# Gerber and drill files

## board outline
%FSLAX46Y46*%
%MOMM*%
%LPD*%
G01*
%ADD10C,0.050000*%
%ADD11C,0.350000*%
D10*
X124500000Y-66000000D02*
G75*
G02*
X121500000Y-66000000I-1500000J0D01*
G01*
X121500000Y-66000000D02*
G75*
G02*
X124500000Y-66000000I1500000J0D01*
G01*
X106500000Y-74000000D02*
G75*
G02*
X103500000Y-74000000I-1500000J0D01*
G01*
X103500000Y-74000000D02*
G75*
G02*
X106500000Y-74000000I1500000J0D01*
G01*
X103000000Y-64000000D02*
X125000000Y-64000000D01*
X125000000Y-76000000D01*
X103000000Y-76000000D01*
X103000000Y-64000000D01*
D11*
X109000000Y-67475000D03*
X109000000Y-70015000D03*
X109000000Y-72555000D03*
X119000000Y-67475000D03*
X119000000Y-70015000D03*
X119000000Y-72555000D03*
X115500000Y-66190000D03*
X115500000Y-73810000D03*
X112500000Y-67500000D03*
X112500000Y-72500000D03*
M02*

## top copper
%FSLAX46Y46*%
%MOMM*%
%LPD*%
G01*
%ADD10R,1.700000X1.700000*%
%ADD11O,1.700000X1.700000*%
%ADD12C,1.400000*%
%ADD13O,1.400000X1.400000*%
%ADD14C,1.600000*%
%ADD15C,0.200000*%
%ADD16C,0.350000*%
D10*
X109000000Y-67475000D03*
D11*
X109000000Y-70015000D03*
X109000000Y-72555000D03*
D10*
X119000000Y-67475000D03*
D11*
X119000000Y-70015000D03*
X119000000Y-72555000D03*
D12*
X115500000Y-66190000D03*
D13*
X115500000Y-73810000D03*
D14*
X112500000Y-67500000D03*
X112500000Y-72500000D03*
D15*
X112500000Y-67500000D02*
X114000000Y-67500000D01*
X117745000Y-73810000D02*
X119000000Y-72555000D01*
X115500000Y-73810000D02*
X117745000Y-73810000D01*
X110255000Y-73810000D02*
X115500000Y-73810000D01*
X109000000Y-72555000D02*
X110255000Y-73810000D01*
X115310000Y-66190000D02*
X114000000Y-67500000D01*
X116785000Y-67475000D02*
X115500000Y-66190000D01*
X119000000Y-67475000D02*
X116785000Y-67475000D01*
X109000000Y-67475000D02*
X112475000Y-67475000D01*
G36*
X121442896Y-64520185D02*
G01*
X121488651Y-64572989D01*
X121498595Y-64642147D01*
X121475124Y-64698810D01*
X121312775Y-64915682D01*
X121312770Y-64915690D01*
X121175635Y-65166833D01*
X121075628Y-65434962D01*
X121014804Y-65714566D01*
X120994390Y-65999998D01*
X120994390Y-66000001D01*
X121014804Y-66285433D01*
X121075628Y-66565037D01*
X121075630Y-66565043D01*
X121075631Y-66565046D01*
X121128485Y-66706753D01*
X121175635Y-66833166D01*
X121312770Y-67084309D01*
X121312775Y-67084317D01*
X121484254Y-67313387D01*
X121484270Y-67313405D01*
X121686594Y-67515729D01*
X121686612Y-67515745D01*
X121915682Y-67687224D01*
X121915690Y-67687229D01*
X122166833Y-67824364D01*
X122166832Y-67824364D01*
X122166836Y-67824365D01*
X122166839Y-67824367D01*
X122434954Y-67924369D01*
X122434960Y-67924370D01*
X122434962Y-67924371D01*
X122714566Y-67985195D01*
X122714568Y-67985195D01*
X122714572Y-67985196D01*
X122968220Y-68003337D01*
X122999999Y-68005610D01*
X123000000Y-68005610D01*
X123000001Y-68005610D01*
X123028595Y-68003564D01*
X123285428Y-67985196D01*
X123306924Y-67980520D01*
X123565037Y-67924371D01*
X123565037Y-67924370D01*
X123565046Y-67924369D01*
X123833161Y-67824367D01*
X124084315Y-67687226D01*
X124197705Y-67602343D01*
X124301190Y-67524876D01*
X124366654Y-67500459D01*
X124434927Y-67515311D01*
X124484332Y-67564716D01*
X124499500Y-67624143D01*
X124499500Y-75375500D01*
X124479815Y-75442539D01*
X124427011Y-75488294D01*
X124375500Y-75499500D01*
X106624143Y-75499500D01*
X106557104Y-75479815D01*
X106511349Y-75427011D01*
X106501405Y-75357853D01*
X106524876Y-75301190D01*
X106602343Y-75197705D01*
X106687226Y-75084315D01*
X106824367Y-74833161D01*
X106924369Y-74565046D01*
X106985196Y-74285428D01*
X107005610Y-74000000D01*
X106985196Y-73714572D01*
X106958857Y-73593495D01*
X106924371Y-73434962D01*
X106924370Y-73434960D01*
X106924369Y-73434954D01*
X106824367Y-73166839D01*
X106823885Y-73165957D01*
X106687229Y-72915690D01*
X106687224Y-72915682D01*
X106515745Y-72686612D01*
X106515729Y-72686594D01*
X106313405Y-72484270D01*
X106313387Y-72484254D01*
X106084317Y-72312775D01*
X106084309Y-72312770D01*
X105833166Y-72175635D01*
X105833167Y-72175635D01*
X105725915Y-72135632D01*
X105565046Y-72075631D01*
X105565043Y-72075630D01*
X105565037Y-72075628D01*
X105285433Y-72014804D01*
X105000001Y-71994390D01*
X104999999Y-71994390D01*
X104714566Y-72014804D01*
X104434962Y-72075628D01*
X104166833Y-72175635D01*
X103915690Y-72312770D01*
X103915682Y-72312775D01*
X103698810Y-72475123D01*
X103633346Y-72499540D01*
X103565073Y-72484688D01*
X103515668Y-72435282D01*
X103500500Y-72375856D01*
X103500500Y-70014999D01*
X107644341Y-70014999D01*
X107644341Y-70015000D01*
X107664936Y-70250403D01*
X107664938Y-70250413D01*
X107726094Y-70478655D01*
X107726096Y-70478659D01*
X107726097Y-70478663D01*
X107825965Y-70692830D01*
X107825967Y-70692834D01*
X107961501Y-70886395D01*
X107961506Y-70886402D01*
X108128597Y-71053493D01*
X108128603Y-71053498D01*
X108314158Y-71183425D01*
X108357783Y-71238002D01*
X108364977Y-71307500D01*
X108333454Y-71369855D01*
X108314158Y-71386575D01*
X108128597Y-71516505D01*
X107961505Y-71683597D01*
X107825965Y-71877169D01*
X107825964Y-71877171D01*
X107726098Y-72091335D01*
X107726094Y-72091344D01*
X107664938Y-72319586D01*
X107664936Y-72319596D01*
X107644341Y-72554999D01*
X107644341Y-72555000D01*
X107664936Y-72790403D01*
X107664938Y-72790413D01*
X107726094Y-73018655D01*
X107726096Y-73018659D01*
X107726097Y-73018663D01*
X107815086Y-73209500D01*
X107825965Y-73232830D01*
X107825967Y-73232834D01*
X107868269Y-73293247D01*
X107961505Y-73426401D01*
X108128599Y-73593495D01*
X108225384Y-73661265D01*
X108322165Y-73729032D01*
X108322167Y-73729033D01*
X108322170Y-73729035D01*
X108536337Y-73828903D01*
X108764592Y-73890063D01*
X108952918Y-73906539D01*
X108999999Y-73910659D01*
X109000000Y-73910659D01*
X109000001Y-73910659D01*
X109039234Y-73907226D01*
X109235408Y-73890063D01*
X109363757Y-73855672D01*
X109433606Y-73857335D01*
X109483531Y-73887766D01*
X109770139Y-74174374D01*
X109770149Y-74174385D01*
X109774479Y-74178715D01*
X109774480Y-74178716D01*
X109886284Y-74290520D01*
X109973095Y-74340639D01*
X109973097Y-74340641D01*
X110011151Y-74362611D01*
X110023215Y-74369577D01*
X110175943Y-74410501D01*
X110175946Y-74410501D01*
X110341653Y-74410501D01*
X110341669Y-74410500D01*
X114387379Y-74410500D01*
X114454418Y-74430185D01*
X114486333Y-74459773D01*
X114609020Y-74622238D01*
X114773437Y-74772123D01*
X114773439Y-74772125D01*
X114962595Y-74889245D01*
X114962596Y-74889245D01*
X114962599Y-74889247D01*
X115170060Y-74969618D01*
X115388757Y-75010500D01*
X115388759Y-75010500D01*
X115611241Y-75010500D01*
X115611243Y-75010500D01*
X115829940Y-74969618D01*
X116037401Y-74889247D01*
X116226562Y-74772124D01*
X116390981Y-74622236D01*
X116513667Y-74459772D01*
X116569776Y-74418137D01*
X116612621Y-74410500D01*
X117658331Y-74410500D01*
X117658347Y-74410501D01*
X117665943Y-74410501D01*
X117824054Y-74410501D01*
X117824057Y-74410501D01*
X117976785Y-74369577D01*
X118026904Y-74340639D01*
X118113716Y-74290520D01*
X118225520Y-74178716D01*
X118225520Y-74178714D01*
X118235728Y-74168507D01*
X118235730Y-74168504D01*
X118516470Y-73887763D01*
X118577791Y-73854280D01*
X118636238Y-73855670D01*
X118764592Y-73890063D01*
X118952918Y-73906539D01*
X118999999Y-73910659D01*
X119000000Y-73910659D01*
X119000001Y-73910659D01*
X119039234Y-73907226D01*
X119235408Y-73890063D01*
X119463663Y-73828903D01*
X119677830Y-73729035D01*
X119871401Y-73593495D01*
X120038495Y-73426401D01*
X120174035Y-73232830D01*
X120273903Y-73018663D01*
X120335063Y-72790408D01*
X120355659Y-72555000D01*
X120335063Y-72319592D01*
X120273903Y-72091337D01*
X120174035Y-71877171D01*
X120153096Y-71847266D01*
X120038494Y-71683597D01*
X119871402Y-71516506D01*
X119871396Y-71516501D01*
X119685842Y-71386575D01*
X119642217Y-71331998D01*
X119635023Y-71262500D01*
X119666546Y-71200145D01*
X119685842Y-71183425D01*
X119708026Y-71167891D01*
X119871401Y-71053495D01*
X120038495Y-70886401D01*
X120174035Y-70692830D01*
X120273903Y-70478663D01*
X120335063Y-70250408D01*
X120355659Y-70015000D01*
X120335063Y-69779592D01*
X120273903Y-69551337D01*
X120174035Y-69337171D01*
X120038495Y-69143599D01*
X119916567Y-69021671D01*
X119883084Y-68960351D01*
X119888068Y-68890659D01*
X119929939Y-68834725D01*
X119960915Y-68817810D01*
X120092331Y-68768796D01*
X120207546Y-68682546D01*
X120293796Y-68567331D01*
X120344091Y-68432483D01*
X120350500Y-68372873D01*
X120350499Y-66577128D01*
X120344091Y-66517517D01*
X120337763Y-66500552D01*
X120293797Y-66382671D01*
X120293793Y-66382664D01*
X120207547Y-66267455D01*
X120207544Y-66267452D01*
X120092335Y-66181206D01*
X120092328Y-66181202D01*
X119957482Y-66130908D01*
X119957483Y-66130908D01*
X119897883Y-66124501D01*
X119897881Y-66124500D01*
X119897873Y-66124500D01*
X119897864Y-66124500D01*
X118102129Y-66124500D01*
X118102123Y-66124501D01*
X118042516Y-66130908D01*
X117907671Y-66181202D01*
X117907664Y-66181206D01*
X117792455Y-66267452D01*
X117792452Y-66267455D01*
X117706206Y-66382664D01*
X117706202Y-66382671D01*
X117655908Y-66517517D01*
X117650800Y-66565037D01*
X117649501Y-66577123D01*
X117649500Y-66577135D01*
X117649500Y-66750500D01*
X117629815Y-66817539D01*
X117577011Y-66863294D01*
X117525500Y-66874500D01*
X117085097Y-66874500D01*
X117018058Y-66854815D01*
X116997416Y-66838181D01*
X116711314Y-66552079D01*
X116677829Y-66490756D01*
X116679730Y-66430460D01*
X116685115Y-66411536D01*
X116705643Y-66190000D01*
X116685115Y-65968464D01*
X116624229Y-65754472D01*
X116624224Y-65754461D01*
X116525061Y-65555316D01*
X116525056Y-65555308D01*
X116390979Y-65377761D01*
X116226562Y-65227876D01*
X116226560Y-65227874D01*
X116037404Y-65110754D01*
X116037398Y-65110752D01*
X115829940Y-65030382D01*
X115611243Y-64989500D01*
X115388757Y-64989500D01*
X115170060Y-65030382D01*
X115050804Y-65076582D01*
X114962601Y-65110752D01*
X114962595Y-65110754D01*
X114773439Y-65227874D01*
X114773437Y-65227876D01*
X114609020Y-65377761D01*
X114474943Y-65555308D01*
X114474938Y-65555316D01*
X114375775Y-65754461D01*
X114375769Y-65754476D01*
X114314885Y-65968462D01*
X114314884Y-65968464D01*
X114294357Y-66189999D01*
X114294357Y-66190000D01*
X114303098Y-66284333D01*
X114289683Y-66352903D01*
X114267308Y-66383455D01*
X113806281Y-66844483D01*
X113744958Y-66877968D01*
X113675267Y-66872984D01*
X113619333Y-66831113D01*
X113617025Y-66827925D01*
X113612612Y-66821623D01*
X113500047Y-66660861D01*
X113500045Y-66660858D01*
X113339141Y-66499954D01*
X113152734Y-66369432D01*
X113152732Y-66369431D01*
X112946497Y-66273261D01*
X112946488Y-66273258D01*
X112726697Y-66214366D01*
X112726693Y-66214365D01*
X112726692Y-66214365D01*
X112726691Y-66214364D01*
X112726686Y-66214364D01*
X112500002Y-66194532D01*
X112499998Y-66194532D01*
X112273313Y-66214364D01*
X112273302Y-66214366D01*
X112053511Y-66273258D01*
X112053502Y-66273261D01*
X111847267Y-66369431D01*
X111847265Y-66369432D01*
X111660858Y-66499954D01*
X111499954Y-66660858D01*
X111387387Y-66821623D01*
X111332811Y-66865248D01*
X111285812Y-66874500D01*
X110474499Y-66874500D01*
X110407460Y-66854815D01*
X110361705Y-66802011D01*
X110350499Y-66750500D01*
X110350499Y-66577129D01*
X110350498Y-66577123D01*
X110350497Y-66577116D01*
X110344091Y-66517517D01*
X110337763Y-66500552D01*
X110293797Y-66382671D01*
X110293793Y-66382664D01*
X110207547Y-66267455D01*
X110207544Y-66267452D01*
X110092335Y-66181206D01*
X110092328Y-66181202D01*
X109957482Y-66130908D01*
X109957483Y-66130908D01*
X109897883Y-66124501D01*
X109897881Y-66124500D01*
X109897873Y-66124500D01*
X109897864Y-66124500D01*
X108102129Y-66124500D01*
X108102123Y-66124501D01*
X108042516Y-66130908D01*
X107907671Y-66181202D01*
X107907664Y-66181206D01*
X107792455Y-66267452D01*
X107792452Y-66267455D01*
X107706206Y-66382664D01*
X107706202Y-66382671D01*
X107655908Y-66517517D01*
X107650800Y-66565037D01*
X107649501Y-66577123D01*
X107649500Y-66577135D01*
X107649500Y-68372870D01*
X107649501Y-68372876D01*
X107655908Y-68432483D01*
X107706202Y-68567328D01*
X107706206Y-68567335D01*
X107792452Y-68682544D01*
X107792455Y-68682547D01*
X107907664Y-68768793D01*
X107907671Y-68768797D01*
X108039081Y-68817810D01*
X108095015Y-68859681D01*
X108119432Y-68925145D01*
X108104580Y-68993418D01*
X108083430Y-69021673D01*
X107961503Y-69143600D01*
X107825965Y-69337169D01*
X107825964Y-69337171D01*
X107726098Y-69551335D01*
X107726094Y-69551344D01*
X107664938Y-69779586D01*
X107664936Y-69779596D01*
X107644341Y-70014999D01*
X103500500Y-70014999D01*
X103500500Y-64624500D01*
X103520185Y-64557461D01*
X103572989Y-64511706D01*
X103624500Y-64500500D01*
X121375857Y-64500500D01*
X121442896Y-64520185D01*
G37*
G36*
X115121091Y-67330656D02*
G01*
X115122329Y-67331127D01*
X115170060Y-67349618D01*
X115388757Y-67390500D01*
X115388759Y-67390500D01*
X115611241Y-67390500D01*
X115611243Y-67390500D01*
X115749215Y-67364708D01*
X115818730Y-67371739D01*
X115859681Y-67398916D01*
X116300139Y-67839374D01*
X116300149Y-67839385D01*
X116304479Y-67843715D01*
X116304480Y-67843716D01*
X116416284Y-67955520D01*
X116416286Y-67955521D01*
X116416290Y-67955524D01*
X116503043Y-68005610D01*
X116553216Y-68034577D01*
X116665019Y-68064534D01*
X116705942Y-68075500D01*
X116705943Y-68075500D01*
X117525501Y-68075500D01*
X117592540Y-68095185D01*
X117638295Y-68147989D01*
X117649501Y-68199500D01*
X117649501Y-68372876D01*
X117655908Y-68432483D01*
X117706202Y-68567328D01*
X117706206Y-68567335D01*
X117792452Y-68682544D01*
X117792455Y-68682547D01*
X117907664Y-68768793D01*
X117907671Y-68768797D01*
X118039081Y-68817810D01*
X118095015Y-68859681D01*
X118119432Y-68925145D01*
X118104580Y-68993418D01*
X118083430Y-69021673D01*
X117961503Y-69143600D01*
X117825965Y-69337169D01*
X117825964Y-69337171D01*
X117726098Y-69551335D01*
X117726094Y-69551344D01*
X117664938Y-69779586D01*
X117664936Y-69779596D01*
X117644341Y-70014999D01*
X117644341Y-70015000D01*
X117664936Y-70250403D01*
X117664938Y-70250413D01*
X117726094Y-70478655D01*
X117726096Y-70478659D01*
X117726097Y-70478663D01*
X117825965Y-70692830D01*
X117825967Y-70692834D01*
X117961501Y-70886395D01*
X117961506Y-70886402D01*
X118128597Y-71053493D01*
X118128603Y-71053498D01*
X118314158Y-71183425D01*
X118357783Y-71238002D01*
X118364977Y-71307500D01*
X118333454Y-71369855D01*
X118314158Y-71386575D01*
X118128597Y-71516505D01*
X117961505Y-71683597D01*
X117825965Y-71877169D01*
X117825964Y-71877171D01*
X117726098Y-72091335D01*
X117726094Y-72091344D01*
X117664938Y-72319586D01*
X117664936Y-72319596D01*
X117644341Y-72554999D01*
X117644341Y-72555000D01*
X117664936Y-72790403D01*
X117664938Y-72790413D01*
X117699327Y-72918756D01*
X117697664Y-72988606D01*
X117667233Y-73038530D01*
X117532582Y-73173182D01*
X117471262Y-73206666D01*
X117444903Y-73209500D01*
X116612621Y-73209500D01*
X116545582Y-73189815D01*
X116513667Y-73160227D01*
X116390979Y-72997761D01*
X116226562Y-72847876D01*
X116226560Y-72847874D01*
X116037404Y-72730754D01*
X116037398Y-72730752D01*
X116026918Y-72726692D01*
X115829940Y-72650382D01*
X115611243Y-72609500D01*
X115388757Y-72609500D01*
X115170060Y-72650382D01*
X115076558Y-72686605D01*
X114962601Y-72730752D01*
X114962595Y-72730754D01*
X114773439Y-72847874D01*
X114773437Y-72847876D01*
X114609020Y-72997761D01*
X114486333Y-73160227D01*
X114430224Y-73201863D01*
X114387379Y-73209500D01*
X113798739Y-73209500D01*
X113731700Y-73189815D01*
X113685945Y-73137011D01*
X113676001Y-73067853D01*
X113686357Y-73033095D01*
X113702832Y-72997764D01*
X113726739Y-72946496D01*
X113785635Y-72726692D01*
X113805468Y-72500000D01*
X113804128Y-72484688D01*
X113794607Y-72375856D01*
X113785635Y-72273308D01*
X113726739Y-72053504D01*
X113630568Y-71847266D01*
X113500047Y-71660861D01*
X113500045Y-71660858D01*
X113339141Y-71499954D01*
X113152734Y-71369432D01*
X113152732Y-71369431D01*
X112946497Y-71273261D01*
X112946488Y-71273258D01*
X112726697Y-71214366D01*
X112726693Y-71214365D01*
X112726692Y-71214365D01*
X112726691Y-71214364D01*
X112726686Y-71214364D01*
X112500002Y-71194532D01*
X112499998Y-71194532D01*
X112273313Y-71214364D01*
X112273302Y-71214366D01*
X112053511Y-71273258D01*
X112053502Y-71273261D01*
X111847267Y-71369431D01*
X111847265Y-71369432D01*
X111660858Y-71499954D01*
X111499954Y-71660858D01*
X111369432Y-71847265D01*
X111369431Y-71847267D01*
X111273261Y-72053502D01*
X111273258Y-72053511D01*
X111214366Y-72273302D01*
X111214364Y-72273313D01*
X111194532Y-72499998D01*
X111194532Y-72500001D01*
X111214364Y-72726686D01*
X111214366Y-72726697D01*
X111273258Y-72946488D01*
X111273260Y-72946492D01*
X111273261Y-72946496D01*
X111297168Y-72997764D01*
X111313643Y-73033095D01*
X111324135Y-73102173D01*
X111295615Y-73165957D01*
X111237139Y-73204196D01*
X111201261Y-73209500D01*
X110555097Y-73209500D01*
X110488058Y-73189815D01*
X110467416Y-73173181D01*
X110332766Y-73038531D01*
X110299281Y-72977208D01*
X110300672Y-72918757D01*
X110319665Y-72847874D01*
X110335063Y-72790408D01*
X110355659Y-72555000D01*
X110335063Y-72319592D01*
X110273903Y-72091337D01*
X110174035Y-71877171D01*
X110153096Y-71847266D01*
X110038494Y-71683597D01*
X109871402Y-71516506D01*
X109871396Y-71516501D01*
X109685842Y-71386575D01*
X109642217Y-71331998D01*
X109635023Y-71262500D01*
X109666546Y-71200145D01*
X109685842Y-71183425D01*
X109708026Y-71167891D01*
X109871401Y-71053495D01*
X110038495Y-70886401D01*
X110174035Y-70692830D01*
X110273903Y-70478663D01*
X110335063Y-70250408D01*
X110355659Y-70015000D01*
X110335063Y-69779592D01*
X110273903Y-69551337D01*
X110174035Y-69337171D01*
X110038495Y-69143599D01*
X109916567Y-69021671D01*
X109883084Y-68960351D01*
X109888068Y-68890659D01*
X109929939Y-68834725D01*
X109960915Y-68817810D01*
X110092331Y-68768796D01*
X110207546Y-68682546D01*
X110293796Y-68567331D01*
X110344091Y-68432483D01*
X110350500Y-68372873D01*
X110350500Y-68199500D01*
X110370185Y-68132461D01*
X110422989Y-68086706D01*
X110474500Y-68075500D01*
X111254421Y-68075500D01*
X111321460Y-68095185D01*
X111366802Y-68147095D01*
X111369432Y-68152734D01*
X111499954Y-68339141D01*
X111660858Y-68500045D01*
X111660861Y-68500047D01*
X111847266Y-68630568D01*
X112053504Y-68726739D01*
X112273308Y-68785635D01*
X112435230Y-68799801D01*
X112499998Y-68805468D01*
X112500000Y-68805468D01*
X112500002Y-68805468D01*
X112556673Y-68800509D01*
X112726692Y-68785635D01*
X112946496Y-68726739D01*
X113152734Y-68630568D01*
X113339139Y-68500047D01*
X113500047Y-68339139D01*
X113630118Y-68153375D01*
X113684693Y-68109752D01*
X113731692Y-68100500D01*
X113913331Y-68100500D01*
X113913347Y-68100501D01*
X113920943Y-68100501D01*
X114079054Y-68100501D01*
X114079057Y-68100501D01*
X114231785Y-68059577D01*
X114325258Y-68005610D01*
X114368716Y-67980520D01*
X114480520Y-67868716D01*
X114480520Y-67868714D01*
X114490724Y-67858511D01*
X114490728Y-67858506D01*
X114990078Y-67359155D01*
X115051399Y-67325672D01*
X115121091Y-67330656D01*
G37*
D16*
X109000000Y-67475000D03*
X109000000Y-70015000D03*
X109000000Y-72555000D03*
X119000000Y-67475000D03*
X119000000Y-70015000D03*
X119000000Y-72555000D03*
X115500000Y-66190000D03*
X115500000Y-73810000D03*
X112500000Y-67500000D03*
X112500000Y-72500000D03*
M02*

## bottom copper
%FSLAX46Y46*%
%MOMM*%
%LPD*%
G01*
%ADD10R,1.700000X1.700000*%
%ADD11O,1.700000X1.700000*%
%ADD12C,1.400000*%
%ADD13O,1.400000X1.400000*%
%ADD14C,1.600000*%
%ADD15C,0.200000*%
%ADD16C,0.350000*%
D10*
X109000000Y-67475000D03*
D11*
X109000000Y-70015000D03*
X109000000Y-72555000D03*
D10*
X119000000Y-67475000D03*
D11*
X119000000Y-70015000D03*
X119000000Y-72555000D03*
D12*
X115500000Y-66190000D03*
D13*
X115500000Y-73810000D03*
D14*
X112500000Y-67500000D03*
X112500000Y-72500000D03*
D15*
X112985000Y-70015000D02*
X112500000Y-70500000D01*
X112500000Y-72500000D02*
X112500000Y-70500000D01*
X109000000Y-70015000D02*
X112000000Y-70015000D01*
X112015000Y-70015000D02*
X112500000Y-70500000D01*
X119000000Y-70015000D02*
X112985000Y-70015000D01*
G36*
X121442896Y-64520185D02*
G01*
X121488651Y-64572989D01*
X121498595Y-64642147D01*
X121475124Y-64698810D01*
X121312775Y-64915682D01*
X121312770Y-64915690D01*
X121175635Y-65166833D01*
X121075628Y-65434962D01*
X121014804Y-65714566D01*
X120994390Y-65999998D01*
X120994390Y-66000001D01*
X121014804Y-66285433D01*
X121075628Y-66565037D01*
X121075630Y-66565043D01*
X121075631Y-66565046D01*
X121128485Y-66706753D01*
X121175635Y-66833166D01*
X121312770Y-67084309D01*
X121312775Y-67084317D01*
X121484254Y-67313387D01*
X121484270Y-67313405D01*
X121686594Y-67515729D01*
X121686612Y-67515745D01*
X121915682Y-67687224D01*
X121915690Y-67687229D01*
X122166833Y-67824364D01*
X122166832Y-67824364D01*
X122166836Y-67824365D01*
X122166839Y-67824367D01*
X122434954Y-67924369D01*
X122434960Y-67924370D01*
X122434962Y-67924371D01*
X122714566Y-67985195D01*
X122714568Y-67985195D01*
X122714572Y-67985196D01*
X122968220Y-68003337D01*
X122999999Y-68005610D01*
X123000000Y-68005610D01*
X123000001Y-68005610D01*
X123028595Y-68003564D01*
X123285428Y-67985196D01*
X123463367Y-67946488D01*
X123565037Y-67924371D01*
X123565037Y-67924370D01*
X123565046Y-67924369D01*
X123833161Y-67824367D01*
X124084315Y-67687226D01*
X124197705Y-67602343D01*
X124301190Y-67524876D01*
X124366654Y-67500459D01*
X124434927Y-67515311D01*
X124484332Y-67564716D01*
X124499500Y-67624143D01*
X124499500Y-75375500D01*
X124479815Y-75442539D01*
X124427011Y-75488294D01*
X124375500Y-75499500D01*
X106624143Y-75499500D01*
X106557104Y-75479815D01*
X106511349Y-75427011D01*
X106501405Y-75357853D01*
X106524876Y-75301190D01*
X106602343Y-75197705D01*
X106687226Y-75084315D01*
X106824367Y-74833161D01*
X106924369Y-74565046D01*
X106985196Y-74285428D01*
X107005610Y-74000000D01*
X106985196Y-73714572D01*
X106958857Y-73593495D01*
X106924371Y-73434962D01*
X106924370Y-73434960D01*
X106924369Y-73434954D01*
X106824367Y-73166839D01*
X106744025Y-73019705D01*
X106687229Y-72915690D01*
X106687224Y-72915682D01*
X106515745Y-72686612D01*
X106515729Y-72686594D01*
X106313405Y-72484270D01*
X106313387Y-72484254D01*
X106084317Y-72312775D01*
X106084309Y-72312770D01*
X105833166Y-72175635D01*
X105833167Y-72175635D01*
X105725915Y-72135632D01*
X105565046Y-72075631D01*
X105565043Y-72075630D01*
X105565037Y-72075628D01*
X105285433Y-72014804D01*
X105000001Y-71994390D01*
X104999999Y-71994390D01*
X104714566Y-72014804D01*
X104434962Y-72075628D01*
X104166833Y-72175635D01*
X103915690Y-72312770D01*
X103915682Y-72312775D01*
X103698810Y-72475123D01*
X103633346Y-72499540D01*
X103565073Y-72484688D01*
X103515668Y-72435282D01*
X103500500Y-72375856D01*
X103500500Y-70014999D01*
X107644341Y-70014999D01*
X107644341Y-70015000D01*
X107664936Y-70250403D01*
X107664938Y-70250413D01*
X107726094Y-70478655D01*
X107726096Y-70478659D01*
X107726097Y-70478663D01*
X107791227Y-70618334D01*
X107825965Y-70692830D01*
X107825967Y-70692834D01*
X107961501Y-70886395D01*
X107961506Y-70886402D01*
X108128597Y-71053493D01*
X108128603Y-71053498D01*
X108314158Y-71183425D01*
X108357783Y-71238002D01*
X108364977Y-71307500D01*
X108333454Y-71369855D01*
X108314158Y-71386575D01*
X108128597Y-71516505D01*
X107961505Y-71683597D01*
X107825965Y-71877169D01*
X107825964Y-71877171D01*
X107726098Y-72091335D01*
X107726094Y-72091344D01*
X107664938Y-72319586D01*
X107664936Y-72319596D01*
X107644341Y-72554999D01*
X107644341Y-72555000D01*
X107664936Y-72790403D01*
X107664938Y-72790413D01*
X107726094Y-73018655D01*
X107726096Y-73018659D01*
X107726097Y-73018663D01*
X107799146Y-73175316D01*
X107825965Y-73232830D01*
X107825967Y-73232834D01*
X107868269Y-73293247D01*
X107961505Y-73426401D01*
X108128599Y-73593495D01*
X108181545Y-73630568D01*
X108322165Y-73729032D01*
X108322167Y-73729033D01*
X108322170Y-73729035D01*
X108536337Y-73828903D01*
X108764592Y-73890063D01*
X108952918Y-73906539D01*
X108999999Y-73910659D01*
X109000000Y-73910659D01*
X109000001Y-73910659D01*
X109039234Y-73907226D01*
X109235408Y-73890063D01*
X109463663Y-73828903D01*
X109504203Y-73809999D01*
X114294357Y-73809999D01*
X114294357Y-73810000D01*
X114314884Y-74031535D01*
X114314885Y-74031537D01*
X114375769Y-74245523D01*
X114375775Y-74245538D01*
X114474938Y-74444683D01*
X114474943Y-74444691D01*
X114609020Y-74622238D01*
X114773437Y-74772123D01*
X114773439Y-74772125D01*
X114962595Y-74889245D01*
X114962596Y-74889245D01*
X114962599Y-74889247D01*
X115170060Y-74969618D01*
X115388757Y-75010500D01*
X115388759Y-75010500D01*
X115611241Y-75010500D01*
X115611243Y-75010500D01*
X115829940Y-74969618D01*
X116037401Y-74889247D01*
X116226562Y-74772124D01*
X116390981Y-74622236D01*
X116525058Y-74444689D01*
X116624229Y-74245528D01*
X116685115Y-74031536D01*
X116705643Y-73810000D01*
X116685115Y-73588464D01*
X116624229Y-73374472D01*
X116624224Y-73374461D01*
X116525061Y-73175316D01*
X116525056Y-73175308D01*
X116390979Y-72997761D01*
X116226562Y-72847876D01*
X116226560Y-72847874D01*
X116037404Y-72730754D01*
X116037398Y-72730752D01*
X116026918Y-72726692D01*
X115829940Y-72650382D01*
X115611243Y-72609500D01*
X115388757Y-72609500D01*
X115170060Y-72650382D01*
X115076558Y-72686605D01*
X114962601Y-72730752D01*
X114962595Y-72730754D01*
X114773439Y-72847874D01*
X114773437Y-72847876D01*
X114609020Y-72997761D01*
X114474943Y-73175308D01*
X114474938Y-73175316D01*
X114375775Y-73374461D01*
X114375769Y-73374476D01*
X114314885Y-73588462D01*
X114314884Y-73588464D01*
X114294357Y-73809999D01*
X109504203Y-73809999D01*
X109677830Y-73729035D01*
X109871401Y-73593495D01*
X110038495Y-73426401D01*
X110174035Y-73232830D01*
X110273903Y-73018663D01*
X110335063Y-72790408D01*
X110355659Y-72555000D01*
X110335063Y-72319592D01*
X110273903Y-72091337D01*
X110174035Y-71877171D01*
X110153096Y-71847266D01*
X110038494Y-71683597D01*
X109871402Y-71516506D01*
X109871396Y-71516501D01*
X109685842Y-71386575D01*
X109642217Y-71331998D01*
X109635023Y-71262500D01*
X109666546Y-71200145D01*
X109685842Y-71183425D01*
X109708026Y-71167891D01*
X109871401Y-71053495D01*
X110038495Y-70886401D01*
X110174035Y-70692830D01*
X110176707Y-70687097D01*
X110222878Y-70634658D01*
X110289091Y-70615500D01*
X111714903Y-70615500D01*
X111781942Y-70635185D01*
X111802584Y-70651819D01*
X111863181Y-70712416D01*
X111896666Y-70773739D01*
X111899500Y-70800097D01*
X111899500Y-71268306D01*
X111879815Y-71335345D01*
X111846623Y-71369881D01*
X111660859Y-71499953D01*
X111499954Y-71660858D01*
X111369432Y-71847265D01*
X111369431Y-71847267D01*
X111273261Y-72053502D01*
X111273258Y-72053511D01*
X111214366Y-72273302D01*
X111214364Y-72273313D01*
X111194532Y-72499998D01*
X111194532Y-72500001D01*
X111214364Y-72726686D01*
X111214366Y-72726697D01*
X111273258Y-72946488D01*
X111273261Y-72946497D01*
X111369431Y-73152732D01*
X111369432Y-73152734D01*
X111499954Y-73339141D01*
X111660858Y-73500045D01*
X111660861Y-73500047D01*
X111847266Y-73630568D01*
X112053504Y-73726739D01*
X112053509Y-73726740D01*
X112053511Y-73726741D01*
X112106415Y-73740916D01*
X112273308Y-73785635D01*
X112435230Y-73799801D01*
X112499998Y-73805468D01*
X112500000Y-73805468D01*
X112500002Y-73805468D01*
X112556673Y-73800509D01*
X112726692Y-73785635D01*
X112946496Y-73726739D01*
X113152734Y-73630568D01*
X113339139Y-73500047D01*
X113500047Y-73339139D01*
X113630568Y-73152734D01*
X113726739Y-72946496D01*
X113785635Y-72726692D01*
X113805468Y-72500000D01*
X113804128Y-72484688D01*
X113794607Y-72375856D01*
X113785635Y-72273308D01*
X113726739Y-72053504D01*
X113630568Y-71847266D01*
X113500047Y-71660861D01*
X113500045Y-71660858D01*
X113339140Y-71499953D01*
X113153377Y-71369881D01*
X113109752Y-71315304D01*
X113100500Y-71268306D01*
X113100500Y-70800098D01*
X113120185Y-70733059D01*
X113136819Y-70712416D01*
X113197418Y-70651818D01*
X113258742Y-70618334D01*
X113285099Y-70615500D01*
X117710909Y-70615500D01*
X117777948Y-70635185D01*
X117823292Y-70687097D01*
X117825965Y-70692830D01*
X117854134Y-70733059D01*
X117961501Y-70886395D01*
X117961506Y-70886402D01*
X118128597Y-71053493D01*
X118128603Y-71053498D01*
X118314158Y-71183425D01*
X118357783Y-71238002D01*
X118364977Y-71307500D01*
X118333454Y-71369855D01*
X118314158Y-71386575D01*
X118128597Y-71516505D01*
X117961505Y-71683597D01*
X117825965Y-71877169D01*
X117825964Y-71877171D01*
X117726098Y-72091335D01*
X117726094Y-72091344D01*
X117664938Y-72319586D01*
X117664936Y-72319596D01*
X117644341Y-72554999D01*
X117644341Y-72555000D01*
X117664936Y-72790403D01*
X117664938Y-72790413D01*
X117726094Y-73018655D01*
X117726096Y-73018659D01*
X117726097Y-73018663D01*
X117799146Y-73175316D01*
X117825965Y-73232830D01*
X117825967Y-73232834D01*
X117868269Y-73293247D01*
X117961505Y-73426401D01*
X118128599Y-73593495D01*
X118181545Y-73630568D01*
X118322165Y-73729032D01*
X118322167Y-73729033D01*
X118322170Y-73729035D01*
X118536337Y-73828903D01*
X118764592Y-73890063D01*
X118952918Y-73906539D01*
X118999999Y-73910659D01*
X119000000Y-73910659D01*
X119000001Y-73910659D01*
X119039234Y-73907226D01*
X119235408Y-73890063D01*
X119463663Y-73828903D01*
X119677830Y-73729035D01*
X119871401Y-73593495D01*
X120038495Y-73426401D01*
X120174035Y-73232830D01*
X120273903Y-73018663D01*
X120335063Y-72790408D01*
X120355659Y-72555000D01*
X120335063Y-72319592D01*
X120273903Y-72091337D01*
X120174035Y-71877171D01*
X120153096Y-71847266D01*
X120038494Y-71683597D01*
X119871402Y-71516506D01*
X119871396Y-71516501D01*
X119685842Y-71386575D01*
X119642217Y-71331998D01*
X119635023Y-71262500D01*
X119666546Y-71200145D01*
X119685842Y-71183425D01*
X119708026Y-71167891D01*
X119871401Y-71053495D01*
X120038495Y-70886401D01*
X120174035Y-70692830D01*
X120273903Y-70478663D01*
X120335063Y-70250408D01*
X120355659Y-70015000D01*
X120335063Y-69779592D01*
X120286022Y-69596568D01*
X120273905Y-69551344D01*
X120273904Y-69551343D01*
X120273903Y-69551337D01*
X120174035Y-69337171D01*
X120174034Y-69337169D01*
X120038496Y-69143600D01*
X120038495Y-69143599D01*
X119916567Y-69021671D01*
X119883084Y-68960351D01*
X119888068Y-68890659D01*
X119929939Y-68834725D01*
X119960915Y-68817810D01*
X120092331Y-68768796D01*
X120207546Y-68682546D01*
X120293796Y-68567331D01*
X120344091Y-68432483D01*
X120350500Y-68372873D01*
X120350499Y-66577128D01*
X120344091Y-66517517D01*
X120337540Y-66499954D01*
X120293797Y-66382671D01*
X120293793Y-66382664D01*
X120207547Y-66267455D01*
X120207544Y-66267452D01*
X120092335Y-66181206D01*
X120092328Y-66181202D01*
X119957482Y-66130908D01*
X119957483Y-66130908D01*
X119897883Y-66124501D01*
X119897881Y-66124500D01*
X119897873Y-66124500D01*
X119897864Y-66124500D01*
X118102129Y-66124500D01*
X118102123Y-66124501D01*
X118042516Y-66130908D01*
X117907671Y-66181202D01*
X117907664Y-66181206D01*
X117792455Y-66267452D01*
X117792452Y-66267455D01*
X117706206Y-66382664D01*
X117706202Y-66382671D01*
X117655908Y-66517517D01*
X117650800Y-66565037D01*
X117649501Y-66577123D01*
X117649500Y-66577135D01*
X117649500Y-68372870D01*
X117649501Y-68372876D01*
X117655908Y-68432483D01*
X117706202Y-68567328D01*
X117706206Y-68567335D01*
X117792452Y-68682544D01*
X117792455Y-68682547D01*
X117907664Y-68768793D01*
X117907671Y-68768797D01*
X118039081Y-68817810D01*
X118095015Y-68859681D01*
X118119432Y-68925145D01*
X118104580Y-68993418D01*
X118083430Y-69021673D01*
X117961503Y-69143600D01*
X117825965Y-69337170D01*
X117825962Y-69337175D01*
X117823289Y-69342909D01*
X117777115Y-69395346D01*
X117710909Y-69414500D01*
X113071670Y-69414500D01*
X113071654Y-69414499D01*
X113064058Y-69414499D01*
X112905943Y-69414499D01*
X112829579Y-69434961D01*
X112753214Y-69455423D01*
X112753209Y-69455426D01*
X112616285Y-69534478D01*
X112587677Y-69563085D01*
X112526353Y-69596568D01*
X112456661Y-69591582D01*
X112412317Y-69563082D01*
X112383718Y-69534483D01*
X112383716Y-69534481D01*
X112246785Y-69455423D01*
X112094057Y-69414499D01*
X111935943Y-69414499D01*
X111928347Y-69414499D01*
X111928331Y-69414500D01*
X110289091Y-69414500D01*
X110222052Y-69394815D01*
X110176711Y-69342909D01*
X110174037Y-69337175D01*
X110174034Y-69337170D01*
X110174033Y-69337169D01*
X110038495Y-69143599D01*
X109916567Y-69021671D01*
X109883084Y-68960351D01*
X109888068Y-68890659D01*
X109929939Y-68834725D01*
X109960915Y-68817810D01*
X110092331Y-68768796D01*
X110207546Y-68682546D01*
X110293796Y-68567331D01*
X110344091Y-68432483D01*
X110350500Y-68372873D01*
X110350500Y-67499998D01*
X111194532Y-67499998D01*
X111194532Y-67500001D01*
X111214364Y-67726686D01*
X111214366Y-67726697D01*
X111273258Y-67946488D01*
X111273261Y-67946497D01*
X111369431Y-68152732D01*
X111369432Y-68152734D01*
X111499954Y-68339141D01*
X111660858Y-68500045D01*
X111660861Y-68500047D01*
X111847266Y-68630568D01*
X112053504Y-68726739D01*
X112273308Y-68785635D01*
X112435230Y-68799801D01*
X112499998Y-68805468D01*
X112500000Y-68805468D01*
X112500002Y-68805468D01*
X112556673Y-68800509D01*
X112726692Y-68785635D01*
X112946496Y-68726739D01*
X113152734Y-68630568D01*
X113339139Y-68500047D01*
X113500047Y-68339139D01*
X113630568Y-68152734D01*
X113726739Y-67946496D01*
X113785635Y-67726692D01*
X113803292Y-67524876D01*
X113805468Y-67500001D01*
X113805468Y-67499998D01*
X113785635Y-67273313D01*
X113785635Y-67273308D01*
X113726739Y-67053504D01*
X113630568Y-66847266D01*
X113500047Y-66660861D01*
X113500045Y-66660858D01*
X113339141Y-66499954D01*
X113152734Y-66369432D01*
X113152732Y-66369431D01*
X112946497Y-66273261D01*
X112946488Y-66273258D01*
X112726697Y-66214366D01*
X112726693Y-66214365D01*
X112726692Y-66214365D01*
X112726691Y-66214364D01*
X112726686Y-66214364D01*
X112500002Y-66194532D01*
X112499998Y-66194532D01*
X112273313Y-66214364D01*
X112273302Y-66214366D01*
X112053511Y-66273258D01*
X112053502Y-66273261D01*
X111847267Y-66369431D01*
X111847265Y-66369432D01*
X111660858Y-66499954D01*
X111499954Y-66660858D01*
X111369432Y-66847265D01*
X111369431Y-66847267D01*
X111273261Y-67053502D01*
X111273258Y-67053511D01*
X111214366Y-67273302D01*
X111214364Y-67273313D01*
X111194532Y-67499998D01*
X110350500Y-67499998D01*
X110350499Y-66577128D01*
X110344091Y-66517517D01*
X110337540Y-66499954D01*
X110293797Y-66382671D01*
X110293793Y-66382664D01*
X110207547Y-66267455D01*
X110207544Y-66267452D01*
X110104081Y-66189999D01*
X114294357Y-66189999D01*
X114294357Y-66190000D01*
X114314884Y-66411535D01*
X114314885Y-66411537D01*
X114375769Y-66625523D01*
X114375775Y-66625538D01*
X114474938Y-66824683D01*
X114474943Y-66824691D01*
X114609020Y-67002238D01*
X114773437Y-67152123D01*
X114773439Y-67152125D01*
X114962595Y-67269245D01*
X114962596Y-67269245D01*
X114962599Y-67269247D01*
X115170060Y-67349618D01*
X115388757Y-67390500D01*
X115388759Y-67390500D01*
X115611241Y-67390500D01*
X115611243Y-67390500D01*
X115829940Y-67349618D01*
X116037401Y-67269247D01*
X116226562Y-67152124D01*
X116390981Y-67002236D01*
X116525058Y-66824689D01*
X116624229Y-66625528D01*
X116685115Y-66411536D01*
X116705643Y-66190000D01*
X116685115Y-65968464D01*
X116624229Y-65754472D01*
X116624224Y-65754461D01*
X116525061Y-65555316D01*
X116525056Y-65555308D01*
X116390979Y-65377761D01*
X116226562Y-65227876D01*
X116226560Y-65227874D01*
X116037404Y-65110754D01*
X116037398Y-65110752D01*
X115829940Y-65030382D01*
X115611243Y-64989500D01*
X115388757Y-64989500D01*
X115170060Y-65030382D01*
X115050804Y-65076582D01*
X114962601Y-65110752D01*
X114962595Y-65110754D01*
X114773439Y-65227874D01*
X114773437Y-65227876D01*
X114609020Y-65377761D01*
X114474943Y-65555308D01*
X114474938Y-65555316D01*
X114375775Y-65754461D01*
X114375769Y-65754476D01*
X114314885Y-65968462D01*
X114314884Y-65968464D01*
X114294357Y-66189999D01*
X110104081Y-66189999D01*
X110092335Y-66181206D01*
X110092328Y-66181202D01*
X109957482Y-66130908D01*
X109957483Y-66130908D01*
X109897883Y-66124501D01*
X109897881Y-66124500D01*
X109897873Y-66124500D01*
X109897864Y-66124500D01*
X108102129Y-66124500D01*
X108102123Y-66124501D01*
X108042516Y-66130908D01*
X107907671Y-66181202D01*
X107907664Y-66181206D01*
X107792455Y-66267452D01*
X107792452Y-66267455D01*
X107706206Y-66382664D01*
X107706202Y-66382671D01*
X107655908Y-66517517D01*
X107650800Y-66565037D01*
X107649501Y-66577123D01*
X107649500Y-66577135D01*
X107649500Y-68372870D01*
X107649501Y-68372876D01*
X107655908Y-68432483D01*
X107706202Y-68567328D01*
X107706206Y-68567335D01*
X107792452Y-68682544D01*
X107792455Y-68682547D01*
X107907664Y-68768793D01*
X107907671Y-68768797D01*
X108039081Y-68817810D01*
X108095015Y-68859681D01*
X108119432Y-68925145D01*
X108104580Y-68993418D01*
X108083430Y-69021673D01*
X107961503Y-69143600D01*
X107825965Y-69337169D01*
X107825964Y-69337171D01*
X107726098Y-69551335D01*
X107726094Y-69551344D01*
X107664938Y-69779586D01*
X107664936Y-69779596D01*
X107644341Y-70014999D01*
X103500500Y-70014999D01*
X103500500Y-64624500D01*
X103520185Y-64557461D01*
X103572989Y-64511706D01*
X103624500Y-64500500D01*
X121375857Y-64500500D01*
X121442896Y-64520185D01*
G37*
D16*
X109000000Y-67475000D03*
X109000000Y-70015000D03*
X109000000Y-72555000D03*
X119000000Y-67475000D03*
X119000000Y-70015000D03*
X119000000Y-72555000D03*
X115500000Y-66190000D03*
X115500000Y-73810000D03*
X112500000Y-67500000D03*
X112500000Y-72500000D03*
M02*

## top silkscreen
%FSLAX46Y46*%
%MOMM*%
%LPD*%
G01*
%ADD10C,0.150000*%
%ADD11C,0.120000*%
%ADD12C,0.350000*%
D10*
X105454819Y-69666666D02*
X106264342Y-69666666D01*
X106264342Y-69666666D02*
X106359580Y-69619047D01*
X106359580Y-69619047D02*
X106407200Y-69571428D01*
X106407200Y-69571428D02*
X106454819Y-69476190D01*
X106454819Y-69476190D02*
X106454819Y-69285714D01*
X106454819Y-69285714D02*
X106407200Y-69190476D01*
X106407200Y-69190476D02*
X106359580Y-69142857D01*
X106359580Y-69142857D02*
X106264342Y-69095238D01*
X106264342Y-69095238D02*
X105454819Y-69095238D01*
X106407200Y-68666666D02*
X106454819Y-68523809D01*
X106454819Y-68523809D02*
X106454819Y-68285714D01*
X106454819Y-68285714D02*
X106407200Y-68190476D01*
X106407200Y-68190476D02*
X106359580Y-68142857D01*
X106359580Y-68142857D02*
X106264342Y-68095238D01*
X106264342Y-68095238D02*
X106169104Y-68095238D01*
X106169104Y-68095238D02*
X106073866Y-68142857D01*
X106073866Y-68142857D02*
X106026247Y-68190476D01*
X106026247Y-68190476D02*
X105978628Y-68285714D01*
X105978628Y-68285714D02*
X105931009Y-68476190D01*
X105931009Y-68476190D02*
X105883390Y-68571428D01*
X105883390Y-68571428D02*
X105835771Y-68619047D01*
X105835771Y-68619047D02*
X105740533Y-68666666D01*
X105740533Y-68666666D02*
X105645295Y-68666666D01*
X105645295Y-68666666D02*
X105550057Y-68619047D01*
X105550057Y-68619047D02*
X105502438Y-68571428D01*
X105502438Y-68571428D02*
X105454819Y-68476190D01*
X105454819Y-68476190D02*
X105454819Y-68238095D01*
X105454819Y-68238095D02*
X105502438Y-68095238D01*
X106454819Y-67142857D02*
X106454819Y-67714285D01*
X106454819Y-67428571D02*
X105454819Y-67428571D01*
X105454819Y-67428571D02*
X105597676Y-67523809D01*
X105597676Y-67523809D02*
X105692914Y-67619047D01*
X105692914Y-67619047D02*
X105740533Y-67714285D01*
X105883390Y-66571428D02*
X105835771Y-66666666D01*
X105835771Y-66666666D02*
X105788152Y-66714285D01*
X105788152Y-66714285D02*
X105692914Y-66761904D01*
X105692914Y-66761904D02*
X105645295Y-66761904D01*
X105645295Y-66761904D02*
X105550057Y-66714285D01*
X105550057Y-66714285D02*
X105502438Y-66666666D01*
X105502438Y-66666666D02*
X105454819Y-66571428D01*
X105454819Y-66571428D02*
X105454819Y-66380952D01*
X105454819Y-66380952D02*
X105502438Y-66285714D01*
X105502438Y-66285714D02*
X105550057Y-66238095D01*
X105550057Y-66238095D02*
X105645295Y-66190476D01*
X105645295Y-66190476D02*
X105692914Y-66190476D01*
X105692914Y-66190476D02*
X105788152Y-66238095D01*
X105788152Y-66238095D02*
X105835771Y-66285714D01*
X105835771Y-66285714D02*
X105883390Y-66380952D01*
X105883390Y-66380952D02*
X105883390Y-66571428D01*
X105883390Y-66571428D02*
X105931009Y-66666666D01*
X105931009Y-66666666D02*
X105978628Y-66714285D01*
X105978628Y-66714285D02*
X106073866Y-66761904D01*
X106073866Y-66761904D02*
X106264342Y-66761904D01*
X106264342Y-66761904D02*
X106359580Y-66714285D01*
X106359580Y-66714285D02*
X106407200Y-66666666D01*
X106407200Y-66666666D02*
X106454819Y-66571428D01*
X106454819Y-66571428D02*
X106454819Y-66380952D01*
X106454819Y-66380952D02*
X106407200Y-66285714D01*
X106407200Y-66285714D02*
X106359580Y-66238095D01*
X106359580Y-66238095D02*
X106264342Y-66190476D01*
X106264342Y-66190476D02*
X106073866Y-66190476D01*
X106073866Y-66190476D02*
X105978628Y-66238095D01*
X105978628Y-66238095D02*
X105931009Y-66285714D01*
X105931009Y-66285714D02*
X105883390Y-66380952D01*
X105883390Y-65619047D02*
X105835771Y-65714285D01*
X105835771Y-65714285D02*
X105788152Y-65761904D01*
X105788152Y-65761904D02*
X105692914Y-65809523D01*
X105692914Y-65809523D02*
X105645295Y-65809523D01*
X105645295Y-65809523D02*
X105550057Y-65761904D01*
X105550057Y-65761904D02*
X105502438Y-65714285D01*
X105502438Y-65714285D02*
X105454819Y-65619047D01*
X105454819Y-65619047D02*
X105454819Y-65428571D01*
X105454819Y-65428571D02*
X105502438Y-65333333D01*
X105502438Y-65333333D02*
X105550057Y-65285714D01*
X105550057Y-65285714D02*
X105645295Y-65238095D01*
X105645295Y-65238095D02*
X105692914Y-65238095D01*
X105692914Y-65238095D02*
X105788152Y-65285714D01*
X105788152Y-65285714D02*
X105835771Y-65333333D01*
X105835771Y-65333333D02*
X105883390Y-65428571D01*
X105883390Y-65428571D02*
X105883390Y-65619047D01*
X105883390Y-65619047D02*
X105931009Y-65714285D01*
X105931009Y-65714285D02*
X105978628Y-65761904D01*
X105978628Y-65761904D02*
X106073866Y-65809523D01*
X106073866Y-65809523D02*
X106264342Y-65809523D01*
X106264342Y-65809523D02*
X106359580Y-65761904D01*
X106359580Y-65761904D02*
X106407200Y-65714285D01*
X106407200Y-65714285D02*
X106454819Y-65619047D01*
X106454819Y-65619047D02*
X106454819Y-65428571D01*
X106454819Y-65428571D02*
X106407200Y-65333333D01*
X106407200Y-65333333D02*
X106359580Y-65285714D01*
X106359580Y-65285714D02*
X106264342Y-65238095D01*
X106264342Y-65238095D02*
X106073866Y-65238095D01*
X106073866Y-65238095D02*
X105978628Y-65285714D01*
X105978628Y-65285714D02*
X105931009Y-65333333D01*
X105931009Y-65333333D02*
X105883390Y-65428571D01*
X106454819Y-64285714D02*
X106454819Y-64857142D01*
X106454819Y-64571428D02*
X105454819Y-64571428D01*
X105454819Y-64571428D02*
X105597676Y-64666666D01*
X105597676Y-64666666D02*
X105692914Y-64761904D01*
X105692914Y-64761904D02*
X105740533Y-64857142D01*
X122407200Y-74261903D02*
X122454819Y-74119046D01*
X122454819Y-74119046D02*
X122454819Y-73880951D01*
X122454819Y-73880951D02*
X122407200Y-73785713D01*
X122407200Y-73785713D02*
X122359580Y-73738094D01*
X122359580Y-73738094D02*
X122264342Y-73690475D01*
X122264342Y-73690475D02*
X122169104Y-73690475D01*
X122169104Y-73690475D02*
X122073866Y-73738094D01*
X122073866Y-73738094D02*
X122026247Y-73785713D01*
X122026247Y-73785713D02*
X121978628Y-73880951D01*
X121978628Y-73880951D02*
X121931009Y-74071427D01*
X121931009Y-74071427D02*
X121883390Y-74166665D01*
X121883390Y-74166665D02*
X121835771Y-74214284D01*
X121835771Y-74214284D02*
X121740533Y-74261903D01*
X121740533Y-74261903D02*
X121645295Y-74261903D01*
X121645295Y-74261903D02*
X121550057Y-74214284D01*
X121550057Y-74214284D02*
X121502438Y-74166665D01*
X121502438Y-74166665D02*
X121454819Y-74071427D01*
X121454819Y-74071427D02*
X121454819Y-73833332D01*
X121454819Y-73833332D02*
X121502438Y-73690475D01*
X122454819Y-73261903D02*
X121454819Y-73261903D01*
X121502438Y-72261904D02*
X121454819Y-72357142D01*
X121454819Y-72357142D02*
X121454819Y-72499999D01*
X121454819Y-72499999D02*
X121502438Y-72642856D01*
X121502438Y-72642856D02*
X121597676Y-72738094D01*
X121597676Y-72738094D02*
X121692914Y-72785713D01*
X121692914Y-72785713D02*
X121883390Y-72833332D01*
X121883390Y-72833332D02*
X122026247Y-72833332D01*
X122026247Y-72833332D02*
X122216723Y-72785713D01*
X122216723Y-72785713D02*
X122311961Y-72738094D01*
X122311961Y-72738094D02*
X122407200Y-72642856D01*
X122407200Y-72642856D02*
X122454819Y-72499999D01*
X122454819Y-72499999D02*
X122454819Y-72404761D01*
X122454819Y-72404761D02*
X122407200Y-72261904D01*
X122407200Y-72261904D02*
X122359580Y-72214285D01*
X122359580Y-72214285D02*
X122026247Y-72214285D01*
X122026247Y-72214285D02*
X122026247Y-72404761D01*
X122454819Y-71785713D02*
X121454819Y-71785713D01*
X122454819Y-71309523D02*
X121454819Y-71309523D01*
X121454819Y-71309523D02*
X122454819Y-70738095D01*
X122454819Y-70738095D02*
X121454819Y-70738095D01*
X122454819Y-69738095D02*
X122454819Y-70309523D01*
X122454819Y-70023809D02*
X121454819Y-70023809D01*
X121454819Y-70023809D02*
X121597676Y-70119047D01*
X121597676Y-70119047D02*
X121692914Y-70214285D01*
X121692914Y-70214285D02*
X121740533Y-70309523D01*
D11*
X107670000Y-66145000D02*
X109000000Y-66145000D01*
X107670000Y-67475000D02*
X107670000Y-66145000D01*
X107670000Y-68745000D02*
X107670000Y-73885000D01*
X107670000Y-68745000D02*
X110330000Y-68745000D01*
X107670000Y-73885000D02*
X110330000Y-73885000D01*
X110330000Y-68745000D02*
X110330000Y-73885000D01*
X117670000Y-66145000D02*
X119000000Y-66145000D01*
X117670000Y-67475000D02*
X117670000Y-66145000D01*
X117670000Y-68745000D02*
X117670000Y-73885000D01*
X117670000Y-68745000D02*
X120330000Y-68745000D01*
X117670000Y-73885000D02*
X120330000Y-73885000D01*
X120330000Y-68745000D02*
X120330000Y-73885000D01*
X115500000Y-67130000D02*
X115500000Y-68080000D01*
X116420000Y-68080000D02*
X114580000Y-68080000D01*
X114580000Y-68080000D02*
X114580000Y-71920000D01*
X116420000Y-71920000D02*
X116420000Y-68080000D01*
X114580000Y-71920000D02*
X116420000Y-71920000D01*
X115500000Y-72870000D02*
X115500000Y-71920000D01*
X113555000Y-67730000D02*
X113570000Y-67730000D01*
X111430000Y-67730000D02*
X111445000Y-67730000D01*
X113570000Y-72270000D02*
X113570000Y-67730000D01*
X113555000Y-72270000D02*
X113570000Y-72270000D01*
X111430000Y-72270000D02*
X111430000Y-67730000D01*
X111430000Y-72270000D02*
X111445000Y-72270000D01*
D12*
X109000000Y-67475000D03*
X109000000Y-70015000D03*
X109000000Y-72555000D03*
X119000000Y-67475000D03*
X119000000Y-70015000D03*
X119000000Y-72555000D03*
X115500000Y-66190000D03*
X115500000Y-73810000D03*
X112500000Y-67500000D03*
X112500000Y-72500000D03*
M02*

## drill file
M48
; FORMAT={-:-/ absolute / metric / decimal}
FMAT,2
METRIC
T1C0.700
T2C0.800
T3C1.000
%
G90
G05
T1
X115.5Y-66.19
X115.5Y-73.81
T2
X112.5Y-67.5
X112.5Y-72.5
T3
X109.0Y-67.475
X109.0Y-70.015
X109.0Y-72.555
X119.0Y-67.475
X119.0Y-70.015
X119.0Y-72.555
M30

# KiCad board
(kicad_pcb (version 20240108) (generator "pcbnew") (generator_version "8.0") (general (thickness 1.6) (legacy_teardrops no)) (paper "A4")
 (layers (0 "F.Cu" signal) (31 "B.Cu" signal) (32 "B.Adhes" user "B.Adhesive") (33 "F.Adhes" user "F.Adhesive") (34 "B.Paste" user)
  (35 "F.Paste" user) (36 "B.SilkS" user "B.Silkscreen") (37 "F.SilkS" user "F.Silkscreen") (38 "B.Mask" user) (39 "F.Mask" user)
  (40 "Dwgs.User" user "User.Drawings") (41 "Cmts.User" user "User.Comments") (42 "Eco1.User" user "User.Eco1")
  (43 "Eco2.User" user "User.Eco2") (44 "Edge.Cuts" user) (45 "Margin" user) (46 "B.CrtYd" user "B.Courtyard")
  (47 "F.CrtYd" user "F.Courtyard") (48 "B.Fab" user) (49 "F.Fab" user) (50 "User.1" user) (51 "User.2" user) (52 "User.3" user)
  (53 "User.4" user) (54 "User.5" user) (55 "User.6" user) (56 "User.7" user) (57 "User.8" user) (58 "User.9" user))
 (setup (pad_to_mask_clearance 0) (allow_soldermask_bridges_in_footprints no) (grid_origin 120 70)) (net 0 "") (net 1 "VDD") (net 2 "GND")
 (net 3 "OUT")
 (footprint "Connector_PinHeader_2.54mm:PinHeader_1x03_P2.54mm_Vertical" (layer "F.Cu") (at 119 67.475)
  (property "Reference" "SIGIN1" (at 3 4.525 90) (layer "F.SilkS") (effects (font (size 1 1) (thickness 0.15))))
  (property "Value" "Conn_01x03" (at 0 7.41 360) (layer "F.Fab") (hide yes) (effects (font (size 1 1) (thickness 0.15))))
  (fp_line (start -1.33 -1.33) (end 0 -1.33) (stroke (width 0.12) (type solid)) (layer "F.SilkS"))
  (fp_line (start -1.33 0) (end -1.33 -1.33) (stroke (width 0.12) (type solid)) (layer "F.SilkS"))
  (fp_line (start -1.33 1.27) (end -1.33 6.41) (stroke (width 0.12) (type solid)) (layer "F.SilkS"))
  (fp_line (start -1.33 1.27) (end 1.33 1.27) (stroke (width 0.12) (type solid)) (layer "F.SilkS"))
  (fp_line (start -1.33 6.41) (end 1.33 6.41) (stroke (width 0.12) (type solid)) (layer "F.SilkS"))
  (fp_line (start 1.33 1.27) (end 1.33 6.41) (stroke (width 0.12) (type solid)) (layer "F.SilkS"))
  (pad "1" thru_hole rect (at 0 0) (size 1.7 1.7) (drill 1) (layers "*.Cu" "*.Mask") (remove_unused_layers no) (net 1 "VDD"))
  (pad "2" thru_hole oval (at 0 2.54) (size 1.7 1.7) (drill 1) (layers "*.Cu" "*.Mask") (remove_unused_layers no) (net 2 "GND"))
  (pad "3" thru_hole oval (at 0 5.08) (size 1.7 1.7) (drill 1) (layers "*.Cu" "*.Mask") (remove_unused_layers no) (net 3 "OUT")))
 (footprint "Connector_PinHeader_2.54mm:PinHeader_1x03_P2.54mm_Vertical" (layer "F.Cu") (at 109 67.475)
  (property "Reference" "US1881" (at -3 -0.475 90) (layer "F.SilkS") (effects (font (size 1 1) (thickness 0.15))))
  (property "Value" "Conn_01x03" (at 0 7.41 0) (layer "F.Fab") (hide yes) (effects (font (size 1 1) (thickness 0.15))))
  (fp_line (start -1.33 -1.33) (end 0 -1.33) (stroke (width 0.12) (type solid)) (layer "F.SilkS"))
  (fp_line (start -1.33 0) (end -1.33 -1.33) (stroke (width 0.12) (type solid)) (layer "F.SilkS"))
  (fp_line (start -1.33 1.27) (end -1.33 6.41) (stroke (width 0.12) (type solid)) (layer "F.SilkS"))
  (fp_line (start -1.33 1.27) (end 1.33 1.27) (stroke (width 0.12) (type solid)) (layer "F.SilkS"))
  (fp_line (start -1.33 6.41) (end 1.33 6.41) (stroke (width 0.12) (type solid)) (layer "F.SilkS"))
  (fp_line (start 1.33 1.27) (end 1.33 6.41) (stroke (width 0.12) (type solid)) (layer "F.SilkS"))
  (pad "1" thru_hole rect (at 0 0) (size 1.7 1.7) (drill 1) (layers "*.Cu" "*.Mask") (remove_unused_layers no) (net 1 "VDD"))
  (pad "2" thru_hole oval (at 0 2.54) (size 1.7 1.7) (drill 1) (layers "*.Cu" "*.Mask") (remove_unused_layers no) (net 2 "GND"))
  (pad "3" thru_hole oval (at 0 5.08) (size 1.7 1.7) (drill 1) (layers "*.Cu" "*.Mask") (remove_unused_layers no) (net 3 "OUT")))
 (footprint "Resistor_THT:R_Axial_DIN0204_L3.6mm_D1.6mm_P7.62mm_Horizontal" (layer "F.Cu") (at 115.5 66.19 -90)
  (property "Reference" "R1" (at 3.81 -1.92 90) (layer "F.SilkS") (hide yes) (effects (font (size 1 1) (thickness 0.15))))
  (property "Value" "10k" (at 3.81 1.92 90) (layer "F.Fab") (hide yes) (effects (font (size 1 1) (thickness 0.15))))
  (fp_line (start 1.89 0.92) (end 5.73 0.92) (stroke (width 0.12) (type solid)) (layer "F.SilkS"))
  (fp_line (start 5.73 0.92) (end 5.73 -0.92) (stroke (width 0.12) (type solid)) (layer "F.SilkS"))
  (fp_line (start 0.94 0) (end 1.89 0) (stroke (width 0.12) (type solid)) (layer "F.SilkS"))
  (fp_line (start 6.68 0) (end 5.73 0) (stroke (width 0.12) (type solid)) (layer "F.SilkS"))
  (fp_line (start 1.89 -0.92) (end 1.89 0.92) (stroke (width 0.12) (type solid)) (layer "F.SilkS"))
  (fp_line (start 5.73 -0.92) (end 1.89 -0.92) (stroke (width 0.12) (type solid)) (layer "F.SilkS"))
  (pad "1" thru_hole circle (at 0 0 270) (size 1.4 1.4) (drill 0.7) (layers "*.Cu" "*.Mask") (remove_unused_layers no) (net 1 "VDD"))
  (pad "2" thru_hole oval (at 7.62 0 270) (size 1.4 1.4) (drill 0.7) (layers "*.Cu" "*.Mask") (remove_unused_layers no) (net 3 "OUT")))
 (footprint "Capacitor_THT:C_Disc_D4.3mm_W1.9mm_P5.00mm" (layer "F.Cu") (at 112.5 72.5 90)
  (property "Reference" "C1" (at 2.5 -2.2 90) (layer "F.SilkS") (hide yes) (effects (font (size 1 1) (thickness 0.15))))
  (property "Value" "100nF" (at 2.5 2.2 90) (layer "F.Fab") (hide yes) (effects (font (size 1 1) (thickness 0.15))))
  (fp_line (start 4.77 -1.07) (end 4.77 -1.055) (stroke (width 0.12) (type solid)) (layer "F.SilkS"))
  (fp_line (start 0.23 -1.07) (end 4.77 -1.07) (stroke (width 0.12) (type solid)) (layer "F.SilkS"))
  (fp_line (start 0.23 -1.07) (end 0.23 -1.055) (stroke (width 0.12) (type solid)) (layer "F.SilkS"))
  (fp_line (start 4.77 1.055) (end 4.77 1.07) (stroke (width 0.12) (type solid)) (layer "F.SilkS"))
  (fp_line (start 0.23 1.055) (end 0.23 1.07) (stroke (width 0.12) (type solid)) (layer "F.SilkS"))
  (fp_line (start 0.23 1.07) (end 4.77 1.07) (stroke (width 0.12) (type solid)) (layer "F.SilkS"))
  (pad "1" thru_hole circle (at 0 0 90) (size 1.6 1.6) (drill 0.8) (layers "*.Cu" "*.Mask") (remove_unused_layers no) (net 2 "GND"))
  (pad "2" thru_hole circle (at 5 0 90) (size 1.6 1.6) (drill 0.8) (layers "*.Cu" "*.Mask") (remove_unused_layers no) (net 1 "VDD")))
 (gr_circle (center 105 74) (end 106.5 74) (stroke (width 0.05) (type default)) (fill none) (layer "Edge.Cuts"))
 (gr_circle (center 123 66) (end 124.5 66) (stroke (width 0.05) (type default)) (fill none) (layer "Edge.Cuts"))
 (gr_rect (start 103 64) (end 125 76) (stroke (width 0.05) (type default)) (fill none) (layer "Edge.Cuts"))
 (segment (start 112.985 70.015) (end 112.5 70.5) (width 0.2) (layer "B.Cu") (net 2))
 (segment (start 112.5 72.5) (end 112.5 70.5) (width 0.2) (layer "B.Cu") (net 2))
 (segment (start 112.015 70.015) (end 112.5 70.5) (width 0.2) (layer "B.Cu") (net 2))
 (segment (start 119 70.015) (end 112.985 70.015) (width 0.2) (layer "B.Cu") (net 2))
 (segment (start 109 70.015) (end 112 70.015) (width 0.2) (layer "B.Cu") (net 2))
 (segment (start 109 67.475) (end 112.475 67.475) (width 0.2) (layer "F.Cu") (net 1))
 (segment (start 119 67.475) (end 116.785 67.475) (width 0.2) (layer "F.Cu") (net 1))
 (segment (start 115.31 66.19) (end 114 67.5) (width 0.2) (layer "F.Cu") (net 1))
 (segment (start 116.785 67.475) (end 115.5 66.19) (width 0.2) (layer "F.Cu") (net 1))
 (segment (start 112.5 67.5) (end 114 67.5) (width 0.2) (layer "F.Cu") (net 1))
 (segment (start 115.5 73.81) (end 117.745 73.81) (width 0.2) (layer "F.Cu") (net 3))
 (segment (start 110.255 73.81) (end 115.5 73.81) (width 0.2) (layer "F.Cu") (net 3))
 (segment (start 117.745 73.81) (end 119 72.555) (width 0.2) (layer "F.Cu") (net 3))
 (segment (start 109 72.555) (end 110.255 73.81) (width 0.2) (layer "F.Cu") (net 3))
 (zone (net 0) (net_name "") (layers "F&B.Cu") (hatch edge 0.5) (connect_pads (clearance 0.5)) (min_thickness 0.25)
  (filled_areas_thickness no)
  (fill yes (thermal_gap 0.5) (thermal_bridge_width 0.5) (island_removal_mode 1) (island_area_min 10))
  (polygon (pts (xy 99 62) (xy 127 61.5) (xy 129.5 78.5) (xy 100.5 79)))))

